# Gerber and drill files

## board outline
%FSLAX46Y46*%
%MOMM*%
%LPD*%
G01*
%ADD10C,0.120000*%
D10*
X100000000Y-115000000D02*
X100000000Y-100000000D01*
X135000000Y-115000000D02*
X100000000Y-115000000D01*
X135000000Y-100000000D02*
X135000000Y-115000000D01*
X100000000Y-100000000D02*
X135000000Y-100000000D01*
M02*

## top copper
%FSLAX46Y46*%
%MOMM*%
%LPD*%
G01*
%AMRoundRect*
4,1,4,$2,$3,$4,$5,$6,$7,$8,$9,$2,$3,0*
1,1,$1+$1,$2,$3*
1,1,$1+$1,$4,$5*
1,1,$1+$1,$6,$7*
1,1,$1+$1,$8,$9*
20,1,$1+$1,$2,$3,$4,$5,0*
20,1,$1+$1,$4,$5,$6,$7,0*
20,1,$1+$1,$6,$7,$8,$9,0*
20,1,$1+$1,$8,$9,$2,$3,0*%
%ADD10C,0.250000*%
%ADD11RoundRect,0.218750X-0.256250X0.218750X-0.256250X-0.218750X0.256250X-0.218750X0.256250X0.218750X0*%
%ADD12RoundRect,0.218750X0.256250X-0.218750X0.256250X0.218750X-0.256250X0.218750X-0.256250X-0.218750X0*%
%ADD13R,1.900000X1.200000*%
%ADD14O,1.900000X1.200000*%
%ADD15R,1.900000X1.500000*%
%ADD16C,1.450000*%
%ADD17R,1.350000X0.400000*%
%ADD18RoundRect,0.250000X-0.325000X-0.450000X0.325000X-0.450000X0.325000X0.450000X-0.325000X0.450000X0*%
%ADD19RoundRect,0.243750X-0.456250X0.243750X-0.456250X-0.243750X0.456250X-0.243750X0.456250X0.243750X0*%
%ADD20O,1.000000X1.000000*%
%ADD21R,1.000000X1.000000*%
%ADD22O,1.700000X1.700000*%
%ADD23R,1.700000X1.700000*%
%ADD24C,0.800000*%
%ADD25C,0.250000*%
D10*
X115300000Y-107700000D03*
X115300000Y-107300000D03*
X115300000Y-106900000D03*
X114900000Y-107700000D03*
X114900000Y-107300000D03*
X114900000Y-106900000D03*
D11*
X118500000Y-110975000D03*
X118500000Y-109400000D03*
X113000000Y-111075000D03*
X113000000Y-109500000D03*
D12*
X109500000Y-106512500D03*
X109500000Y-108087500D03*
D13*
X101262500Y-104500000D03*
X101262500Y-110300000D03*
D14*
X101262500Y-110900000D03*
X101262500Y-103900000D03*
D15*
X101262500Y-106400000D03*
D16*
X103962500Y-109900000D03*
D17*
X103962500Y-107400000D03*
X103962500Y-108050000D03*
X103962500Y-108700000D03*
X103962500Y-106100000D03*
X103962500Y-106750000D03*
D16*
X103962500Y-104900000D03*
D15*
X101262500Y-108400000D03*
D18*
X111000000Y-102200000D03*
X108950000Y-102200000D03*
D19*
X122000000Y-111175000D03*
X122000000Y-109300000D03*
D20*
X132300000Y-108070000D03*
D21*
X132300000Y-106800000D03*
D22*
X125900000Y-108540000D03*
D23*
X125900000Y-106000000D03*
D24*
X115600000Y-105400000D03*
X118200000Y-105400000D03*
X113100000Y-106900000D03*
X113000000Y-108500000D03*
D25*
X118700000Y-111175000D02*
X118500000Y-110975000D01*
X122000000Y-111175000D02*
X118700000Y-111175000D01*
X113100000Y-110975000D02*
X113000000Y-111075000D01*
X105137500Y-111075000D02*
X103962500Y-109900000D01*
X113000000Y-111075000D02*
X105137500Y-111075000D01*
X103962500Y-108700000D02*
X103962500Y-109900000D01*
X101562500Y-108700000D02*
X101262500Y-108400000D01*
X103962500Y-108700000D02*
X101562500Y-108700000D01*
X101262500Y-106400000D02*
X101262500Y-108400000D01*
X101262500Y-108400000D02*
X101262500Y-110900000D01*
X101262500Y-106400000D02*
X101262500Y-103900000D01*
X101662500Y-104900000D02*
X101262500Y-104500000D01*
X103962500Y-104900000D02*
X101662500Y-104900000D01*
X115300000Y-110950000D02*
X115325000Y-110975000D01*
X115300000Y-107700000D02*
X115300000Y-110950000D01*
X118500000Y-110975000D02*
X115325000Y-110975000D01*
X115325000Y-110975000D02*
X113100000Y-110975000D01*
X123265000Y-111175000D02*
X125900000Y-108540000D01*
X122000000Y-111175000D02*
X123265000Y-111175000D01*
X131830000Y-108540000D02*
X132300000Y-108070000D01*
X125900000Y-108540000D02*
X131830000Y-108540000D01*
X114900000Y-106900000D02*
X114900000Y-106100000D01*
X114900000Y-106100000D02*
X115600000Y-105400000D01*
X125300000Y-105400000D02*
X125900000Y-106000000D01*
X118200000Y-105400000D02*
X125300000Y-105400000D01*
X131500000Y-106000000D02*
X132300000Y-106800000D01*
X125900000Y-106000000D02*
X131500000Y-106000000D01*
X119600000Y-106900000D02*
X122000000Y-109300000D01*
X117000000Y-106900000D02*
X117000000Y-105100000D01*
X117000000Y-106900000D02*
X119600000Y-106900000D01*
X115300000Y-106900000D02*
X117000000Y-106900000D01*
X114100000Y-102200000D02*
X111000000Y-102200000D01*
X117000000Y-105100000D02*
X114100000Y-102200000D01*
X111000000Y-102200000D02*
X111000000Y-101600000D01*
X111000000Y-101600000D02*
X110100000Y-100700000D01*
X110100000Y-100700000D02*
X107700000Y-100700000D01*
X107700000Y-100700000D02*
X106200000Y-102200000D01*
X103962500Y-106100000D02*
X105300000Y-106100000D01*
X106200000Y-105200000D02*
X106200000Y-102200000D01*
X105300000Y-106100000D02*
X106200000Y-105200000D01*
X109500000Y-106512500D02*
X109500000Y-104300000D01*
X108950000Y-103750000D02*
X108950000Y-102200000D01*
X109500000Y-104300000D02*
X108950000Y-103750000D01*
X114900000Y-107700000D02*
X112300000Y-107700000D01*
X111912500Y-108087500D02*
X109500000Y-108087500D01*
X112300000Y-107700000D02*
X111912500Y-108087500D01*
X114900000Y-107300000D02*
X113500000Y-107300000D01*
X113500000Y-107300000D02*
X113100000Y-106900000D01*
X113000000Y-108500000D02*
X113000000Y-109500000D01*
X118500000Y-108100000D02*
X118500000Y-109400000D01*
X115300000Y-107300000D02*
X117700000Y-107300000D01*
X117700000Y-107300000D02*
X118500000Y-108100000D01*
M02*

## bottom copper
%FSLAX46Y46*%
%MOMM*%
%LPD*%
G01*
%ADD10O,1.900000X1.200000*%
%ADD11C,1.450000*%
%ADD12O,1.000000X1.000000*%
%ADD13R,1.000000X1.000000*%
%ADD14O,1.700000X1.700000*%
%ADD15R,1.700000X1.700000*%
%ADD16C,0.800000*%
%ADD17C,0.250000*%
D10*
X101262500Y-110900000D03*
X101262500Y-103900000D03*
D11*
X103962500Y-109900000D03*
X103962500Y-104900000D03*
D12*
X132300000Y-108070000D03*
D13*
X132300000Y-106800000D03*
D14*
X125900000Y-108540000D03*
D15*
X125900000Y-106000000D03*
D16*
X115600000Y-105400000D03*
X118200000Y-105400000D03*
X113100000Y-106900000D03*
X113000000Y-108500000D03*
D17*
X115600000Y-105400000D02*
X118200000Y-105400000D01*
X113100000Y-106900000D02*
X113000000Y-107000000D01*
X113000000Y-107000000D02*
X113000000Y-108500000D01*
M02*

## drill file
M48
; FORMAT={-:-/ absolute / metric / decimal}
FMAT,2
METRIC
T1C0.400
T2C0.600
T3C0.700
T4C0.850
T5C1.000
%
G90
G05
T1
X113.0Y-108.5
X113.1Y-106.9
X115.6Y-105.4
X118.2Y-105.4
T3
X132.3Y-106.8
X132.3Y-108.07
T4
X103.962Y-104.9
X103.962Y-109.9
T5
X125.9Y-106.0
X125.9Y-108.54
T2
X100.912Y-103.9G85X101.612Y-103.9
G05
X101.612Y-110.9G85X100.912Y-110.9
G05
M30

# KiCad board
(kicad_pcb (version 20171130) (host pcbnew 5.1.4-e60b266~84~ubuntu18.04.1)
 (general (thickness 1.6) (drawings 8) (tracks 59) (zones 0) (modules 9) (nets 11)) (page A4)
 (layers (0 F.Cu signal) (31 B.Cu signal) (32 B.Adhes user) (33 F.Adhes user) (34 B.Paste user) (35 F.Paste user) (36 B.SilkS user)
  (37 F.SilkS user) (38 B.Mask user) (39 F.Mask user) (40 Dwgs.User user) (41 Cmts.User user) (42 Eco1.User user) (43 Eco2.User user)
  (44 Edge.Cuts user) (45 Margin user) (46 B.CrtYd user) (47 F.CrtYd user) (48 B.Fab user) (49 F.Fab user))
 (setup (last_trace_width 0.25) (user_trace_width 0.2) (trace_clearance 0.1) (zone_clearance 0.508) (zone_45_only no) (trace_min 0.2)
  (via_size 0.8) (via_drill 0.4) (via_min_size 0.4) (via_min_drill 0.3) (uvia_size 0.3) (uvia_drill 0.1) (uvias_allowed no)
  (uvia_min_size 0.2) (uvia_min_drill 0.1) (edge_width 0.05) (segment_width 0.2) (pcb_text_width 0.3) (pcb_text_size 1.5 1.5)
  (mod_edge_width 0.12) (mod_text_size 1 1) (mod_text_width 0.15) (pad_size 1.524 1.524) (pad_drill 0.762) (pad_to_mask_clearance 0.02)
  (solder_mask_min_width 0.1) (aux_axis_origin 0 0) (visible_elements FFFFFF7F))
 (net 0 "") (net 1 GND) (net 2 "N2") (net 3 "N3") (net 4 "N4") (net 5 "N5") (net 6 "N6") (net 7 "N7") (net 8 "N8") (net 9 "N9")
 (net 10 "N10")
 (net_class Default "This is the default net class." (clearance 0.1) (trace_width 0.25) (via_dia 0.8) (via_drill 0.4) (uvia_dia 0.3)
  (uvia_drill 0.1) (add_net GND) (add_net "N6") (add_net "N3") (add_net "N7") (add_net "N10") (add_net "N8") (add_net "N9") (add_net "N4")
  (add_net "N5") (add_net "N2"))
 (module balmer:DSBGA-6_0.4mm (layer F.Cu) (at 115.1 107.3)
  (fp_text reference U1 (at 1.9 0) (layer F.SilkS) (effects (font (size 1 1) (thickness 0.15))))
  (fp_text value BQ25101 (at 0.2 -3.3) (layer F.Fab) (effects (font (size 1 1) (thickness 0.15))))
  (pad C2 smd circle (at 0.2 0.4) (size 0.25 0.25) (layers F.Cu F.Paste F.Mask) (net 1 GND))
  (pad B2 smd circle (at 0.2 0) (size 0.25 0.25) (layers F.Cu F.Paste F.Mask) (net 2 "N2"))
  (pad A2 smd circle (at 0.2 -0.4) (size 0.25 0.25) (layers F.Cu F.Paste F.Mask) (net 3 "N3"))
  (pad C1 smd circle (at -0.2 0.4) (size 0.25 0.25) (layers F.Cu F.Paste F.Mask) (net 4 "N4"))
  (pad B1 smd circle (at -0.2 0) (size 0.25 0.25) (layers F.Cu F.Paste F.Mask) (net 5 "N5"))
  (pad A1 smd circle (at -0.2 -0.4) (size 0.25 0.25) (layers F.Cu F.Paste F.Mask) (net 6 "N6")))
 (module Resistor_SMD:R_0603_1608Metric (layer F.Cu) (at 118.5 110.1875 270)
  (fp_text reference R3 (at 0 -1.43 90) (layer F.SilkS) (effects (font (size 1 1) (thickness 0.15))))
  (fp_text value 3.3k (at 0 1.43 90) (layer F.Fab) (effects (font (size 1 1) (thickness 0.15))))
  (pad 2 smd roundrect (at 0.7875 0 270) (size 0.875 0.95) (layers F.Cu F.Paste F.Mask) (roundrect_rratio 0.25) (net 1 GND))
  (pad 1 smd roundrect (at -0.7875 0 270) (size 0.875 0.95) (layers F.Cu F.Paste F.Mask) (roundrect_rratio 0.25) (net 2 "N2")))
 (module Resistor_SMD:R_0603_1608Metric (layer F.Cu) (at 113 110.2875 270)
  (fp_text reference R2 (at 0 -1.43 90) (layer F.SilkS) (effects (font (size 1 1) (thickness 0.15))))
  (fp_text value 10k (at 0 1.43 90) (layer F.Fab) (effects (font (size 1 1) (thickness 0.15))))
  (pad 2 smd roundrect (at 0.7875 0 270) (size 0.875 0.95) (layers F.Cu F.Paste F.Mask) (roundrect_rratio 0.25) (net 1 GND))
  (pad 1 smd roundrect (at -0.7875 0 270) (size 0.875 0.95) (layers F.Cu F.Paste F.Mask) (roundrect_rratio 0.25) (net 5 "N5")))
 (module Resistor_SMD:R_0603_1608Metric (layer F.Cu) (at 109.5 107.3 90)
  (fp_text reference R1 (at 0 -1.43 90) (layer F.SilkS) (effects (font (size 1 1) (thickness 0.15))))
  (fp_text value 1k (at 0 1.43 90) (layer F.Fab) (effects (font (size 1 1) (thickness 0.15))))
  (pad 2 smd roundrect (at 0.7875 0 90) (size 0.875 0.95) (layers F.Cu F.Paste F.Mask) (roundrect_rratio 0.25) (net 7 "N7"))
  (pad 1 smd roundrect (at -0.7875 0 90) (size 0.875 0.95) (layers F.Cu F.Paste F.Mask) (roundrect_rratio 0.25) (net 4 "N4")))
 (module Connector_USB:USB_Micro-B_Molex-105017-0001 (layer F.Cu) (at 102.5 107.4 270)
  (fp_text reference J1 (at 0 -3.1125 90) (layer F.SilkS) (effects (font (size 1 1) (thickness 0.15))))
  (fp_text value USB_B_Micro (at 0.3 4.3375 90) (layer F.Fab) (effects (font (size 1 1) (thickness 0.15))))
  (pad 6 smd rect (at -2.9 1.2375 270) (size 1.2 1.9) (layers F.Cu F.Mask) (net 1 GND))
  (pad 6 smd rect (at 2.9 1.2375 270) (size 1.2 1.9) (layers F.Cu F.Mask) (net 1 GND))
  (pad 6 thru_hole oval (at 3.5 1.2375 270) (size 1.2 1.9) (drill oval 0.6 1.3) (layers *.Cu *.Mask) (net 1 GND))
  (pad 6 thru_hole oval (at -3.5 1.2375 90) (size 1.2 1.9) (drill oval 0.6 1.3) (layers *.Cu *.Mask) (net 1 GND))
  (pad 6 smd rect (at -1 1.2375 270) (size 1.5 1.9) (layers F.Cu F.Paste F.Mask) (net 1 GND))
  (pad 6 thru_hole circle (at 2.5 -1.4625 270) (size 1.45 1.45) (drill 0.85) (layers *.Cu *.Mask) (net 1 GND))
  (pad 3 smd rect (at 0 -1.4625 270) (size 0.4 1.35) (layers F.Cu F.Paste F.Mask) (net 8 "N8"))
  (pad 4 smd rect (at 0.65 -1.4625 270) (size 0.4 1.35) (layers F.Cu F.Paste F.Mask) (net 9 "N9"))
  (pad 5 smd rect (at 1.3 -1.4625 270) (size 0.4 1.35) (layers F.Cu F.Paste F.Mask) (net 1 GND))
  (pad 1 smd rect (at -1.3 -1.4625 270) (size 0.4 1.35) (layers F.Cu F.Paste F.Mask) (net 3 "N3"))
  (pad 2 smd rect (at -0.65 -1.4625 270) (size 0.4 1.35) (layers F.Cu F.Paste F.Mask) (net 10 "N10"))
  (pad 6 thru_hole circle (at -2.5 -1.4625 270) (size 1.45 1.45) (drill 0.85) (layers *.Cu *.Mask) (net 1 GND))
  (pad 6 smd rect (at 1 1.2375 270) (size 1.5 1.9) (layers F.Cu F.Paste F.Mask) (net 1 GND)))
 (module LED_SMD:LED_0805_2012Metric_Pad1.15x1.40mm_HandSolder (layer F.Cu) (at 109.975 102.2)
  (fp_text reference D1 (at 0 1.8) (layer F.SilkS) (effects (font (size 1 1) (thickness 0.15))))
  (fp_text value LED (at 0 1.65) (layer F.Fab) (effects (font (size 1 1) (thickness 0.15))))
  (pad 2 smd roundrect (at 1.025 0) (size 1.15 1.4) (layers F.Cu F.Paste F.Mask) (roundrect_rratio 0.217391) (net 3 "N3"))
  (pad 1 smd roundrect (at -1.025 0) (size 1.15 1.4) (layers F.Cu F.Paste F.Mask) (roundrect_rratio 0.217391) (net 7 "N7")))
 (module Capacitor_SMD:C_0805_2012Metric (layer F.Cu) (at 122 110.2375 270)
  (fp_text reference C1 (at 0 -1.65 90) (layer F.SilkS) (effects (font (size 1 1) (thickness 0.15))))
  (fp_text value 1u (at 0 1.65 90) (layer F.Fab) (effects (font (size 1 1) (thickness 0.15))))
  (pad 2 smd roundrect (at 0.9375 0 270) (size 0.975 1.4) (layers F.Cu F.Paste F.Mask) (roundrect_rratio 0.25) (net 1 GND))
  (pad 1 smd roundrect (at -0.9375 0 270) (size 0.975 1.4) (layers F.Cu F.Paste F.Mask) (roundrect_rratio 0.25) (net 3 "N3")))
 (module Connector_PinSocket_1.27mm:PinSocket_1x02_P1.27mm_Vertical (layer F.Cu) (at 132.3 106.8)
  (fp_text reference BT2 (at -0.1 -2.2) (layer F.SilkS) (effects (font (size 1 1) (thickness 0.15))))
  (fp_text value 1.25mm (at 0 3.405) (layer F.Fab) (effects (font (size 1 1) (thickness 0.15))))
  (pad 2 thru_hole oval (at 0 1.27) (size 1 1) (drill 0.7) (layers *.Cu *.Mask) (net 1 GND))
  (pad 1 thru_hole rect (at 0 0) (size 1 1) (drill 0.7) (layers *.Cu *.Mask) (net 6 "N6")))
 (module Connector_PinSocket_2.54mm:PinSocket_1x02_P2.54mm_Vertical (layer F.Cu) (at 125.9 106)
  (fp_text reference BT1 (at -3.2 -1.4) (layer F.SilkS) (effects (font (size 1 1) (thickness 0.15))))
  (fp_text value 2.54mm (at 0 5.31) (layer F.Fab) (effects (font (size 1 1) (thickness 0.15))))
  (pad 2 thru_hole oval (at 0 2.54) (size 1.7 1.7) (drill 1) (layers *.Cu *.Mask) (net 1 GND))
  (pad 1 thru_hole rect (at 0 0) (size 1.7 1.7) (drill 1) (layers *.Cu *.Mask) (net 6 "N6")))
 (gr_line (start 100 115) (end 100 100) (layer Edge.Cuts) (width 0.12))
 (gr_line (start 135 115) (end 100 115) (layer Edge.Cuts) (width 0.12))
 (gr_line (start 135 100) (end 135 115) (layer Edge.Cuts) (width 0.12))
 (gr_line (start 100 100) (end 135 100) (layer Edge.Cuts) (width 0.12))
 (segment (start 118.7 111.175) (end 118.5 110.975) (width 0.25) (layer F.Cu) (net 1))
 (segment (start 122 111.175) (end 118.7 111.175) (width 0.25) (layer F.Cu) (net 1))
 (segment (start 113.1 110.975) (end 113 111.075) (width 0.25) (layer F.Cu) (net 1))
 (segment (start 105.1375 111.075) (end 103.9625 109.9) (width 0.25) (layer F.Cu) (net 1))
 (segment (start 113 111.075) (end 105.1375 111.075) (width 0.25) (layer F.Cu) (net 1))
 (segment (start 103.9625 108.7) (end 103.9625 109.9) (width 0.25) (layer F.Cu) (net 1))
 (segment (start 101.5625 108.7) (end 101.2625 108.4) (width 0.25) (layer F.Cu) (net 1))
 (segment (start 103.9625 108.7) (end 101.5625 108.7) (width 0.25) (layer F.Cu) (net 1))
 (segment (start 101.2625 106.4) (end 101.2625 108.4) (width 0.25) (layer F.Cu) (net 1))
 (segment (start 101.2625 108.4) (end 101.2625 110.9) (width 0.25) (layer F.Cu) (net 1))
 (segment (start 101.2625 106.4) (end 101.2625 103.9) (width 0.25) (layer F.Cu) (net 1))
 (segment (start 101.6625 104.9) (end 101.2625 104.5) (width 0.25) (layer F.Cu) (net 1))
 (segment (start 103.9625 104.9) (end 101.6625 104.9) (width 0.25) (layer F.Cu) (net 1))
 (segment (start 115.3 110.95) (end 115.325 110.975) (width 0.25) (layer F.Cu) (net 1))
 (segment (start 115.3 107.7) (end 115.3 110.95) (width 0.25) (layer F.Cu) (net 1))
 (segment (start 118.5 110.975) (end 115.325 110.975) (width 0.25) (layer F.Cu) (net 1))
 (segment (start 115.325 110.975) (end 113.1 110.975) (width 0.25) (layer F.Cu) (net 1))
 (segment (start 123.265 111.175) (end 125.9 108.54) (width 0.25) (layer F.Cu) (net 1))
 (segment (start 122 111.175) (end 123.265 111.175) (width 0.25) (layer F.Cu) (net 1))
 (segment (start 131.83 108.54) (end 132.3 108.07) (width 0.25) (layer F.Cu) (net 1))
 (segment (start 125.9 108.54) (end 131.83 108.54) (width 0.25) (layer F.Cu) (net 1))
 (via (at 115.6 105.4) (size 0.8) (drill 0.4) (layers F.Cu B.Cu) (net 6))
 (segment (start 114.9 106.9) (end 114.9 106.1) (width 0.25) (layer F.Cu) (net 6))
 (segment (start 114.9 106.1) (end 115.6 105.4) (width 0.25) (layer F.Cu) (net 6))
 (via (at 118.2 105.4) (size 0.8) (drill 0.4) (layers F.Cu B.Cu) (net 6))
 (segment (start 115.6 105.4) (end 118.2 105.4) (width 0.25) (layer B.Cu) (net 6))
 (segment (start 125.3 105.4) (end 125.9 106) (width 0.25) (layer F.Cu) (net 6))
 (segment (start 118.2 105.4) (end 125.3 105.4) (width 0.25) (layer F.Cu) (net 6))
 (segment (start 131.5 106) (end 132.3 106.8) (width 0.25) (layer F.Cu) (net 6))
 (segment (start 125.9 106) (end 131.5 106) (width 0.25) (layer F.Cu) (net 6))
 (segment (start 119.6 106.9) (end 122 109.3) (width 0.25) (layer F.Cu) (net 3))
 (segment (start 117 106.9) (end 117 105.1) (width 0.25) (layer F.Cu) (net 3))
 (segment (start 117 106.9) (end 119.6 106.9) (width 0.25) (layer F.Cu) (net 3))
 (segment (start 115.3 106.9) (end 117 106.9) (width 0.25) (layer F.Cu) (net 3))
 (segment (start 114.1 102.2) (end 111 102.2) (width 0.25) (layer F.Cu) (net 3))
 (segment (start 117 105.1) (end 114.1 102.2) (width 0.25) (layer F.Cu) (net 3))
 (segment (start 111 102.2) (end 111 101.6) (width 0.25) (layer F.Cu) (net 3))
 (segment (start 111 101.6) (end 110.1 100.7) (width 0.25) (layer F.Cu) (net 3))
 (segment (start 110.1 100.7) (end 107.7 100.7) (width 0.25) (layer F.Cu) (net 3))
 (segment (start 107.7 100.7) (end 106.2 102.2) (width 0.25) (layer F.Cu) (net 3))
 (segment (start 103.9625 106.1) (end 105.3 106.1) (width 0.25) (layer F.Cu) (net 3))
 (segment (start 106.2 105.2) (end 106.2 102.2) (width 0.25) (layer F.Cu) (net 3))
 (segment (start 105.3 106.1) (end 106.2 105.2) (width 0.25) (layer F.Cu) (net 3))
 (segment (start 109.5 106.5125) (end 109.5 104.3) (width 0.25) (layer F.Cu) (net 7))
 (segment (start 108.95 103.75) (end 108.95 102.2) (width 0.25) (layer F.Cu) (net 7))
 (segment (start 109.5 104.3) (end 108.95 103.75) (width 0.25) (layer F.Cu) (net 7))
 (segment (start 114.9 107.7) (end 112.3 107.7) (width 0.25) (layer F.Cu) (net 4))
 (segment (start 111.9125 108.0875) (end 109.5 108.0875) (width 0.25) (layer F.Cu) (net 4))
 (segment (start 112.3 107.7) (end 111.9125 108.0875) (width 0.25) (layer F.Cu) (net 4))
 (via (at 113.1 106.9) (size 0.8) (drill 0.4) (layers F.Cu B.Cu) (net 5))
 (segment (start 114.9 107.3) (end 113.5 107.3) (width 0.25) (layer F.Cu) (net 5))
 (segment (start 113.5 107.3) (end 113.1 106.9) (width 0.25) (layer F.Cu) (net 5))
 (via (at 113 108.5) (size 0.8) (drill 0.4) (layers F.Cu B.Cu) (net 5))
 (segment (start 113.1 106.9) (end 113 107) (width 0.25) (layer B.Cu) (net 5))
 (segment (start 113 107) (end 113 108.5) (width 0.25) (layer B.Cu) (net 5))
 (segment (start 113 108.5) (end 113 109.5) (width 0.25) (layer F.Cu) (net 5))
 (segment (start 118.5 108.1) (end 118.5 109.4) (width 0.25) (layer F.Cu) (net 2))
 (segment (start 115.3 107.3) (end 117.7 107.3) (width 0.25) (layer F.Cu) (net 2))
 (segment (start 117.7 107.3) (end 118.5 108.1) (width 0.25) (layer F.Cu) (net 2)))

